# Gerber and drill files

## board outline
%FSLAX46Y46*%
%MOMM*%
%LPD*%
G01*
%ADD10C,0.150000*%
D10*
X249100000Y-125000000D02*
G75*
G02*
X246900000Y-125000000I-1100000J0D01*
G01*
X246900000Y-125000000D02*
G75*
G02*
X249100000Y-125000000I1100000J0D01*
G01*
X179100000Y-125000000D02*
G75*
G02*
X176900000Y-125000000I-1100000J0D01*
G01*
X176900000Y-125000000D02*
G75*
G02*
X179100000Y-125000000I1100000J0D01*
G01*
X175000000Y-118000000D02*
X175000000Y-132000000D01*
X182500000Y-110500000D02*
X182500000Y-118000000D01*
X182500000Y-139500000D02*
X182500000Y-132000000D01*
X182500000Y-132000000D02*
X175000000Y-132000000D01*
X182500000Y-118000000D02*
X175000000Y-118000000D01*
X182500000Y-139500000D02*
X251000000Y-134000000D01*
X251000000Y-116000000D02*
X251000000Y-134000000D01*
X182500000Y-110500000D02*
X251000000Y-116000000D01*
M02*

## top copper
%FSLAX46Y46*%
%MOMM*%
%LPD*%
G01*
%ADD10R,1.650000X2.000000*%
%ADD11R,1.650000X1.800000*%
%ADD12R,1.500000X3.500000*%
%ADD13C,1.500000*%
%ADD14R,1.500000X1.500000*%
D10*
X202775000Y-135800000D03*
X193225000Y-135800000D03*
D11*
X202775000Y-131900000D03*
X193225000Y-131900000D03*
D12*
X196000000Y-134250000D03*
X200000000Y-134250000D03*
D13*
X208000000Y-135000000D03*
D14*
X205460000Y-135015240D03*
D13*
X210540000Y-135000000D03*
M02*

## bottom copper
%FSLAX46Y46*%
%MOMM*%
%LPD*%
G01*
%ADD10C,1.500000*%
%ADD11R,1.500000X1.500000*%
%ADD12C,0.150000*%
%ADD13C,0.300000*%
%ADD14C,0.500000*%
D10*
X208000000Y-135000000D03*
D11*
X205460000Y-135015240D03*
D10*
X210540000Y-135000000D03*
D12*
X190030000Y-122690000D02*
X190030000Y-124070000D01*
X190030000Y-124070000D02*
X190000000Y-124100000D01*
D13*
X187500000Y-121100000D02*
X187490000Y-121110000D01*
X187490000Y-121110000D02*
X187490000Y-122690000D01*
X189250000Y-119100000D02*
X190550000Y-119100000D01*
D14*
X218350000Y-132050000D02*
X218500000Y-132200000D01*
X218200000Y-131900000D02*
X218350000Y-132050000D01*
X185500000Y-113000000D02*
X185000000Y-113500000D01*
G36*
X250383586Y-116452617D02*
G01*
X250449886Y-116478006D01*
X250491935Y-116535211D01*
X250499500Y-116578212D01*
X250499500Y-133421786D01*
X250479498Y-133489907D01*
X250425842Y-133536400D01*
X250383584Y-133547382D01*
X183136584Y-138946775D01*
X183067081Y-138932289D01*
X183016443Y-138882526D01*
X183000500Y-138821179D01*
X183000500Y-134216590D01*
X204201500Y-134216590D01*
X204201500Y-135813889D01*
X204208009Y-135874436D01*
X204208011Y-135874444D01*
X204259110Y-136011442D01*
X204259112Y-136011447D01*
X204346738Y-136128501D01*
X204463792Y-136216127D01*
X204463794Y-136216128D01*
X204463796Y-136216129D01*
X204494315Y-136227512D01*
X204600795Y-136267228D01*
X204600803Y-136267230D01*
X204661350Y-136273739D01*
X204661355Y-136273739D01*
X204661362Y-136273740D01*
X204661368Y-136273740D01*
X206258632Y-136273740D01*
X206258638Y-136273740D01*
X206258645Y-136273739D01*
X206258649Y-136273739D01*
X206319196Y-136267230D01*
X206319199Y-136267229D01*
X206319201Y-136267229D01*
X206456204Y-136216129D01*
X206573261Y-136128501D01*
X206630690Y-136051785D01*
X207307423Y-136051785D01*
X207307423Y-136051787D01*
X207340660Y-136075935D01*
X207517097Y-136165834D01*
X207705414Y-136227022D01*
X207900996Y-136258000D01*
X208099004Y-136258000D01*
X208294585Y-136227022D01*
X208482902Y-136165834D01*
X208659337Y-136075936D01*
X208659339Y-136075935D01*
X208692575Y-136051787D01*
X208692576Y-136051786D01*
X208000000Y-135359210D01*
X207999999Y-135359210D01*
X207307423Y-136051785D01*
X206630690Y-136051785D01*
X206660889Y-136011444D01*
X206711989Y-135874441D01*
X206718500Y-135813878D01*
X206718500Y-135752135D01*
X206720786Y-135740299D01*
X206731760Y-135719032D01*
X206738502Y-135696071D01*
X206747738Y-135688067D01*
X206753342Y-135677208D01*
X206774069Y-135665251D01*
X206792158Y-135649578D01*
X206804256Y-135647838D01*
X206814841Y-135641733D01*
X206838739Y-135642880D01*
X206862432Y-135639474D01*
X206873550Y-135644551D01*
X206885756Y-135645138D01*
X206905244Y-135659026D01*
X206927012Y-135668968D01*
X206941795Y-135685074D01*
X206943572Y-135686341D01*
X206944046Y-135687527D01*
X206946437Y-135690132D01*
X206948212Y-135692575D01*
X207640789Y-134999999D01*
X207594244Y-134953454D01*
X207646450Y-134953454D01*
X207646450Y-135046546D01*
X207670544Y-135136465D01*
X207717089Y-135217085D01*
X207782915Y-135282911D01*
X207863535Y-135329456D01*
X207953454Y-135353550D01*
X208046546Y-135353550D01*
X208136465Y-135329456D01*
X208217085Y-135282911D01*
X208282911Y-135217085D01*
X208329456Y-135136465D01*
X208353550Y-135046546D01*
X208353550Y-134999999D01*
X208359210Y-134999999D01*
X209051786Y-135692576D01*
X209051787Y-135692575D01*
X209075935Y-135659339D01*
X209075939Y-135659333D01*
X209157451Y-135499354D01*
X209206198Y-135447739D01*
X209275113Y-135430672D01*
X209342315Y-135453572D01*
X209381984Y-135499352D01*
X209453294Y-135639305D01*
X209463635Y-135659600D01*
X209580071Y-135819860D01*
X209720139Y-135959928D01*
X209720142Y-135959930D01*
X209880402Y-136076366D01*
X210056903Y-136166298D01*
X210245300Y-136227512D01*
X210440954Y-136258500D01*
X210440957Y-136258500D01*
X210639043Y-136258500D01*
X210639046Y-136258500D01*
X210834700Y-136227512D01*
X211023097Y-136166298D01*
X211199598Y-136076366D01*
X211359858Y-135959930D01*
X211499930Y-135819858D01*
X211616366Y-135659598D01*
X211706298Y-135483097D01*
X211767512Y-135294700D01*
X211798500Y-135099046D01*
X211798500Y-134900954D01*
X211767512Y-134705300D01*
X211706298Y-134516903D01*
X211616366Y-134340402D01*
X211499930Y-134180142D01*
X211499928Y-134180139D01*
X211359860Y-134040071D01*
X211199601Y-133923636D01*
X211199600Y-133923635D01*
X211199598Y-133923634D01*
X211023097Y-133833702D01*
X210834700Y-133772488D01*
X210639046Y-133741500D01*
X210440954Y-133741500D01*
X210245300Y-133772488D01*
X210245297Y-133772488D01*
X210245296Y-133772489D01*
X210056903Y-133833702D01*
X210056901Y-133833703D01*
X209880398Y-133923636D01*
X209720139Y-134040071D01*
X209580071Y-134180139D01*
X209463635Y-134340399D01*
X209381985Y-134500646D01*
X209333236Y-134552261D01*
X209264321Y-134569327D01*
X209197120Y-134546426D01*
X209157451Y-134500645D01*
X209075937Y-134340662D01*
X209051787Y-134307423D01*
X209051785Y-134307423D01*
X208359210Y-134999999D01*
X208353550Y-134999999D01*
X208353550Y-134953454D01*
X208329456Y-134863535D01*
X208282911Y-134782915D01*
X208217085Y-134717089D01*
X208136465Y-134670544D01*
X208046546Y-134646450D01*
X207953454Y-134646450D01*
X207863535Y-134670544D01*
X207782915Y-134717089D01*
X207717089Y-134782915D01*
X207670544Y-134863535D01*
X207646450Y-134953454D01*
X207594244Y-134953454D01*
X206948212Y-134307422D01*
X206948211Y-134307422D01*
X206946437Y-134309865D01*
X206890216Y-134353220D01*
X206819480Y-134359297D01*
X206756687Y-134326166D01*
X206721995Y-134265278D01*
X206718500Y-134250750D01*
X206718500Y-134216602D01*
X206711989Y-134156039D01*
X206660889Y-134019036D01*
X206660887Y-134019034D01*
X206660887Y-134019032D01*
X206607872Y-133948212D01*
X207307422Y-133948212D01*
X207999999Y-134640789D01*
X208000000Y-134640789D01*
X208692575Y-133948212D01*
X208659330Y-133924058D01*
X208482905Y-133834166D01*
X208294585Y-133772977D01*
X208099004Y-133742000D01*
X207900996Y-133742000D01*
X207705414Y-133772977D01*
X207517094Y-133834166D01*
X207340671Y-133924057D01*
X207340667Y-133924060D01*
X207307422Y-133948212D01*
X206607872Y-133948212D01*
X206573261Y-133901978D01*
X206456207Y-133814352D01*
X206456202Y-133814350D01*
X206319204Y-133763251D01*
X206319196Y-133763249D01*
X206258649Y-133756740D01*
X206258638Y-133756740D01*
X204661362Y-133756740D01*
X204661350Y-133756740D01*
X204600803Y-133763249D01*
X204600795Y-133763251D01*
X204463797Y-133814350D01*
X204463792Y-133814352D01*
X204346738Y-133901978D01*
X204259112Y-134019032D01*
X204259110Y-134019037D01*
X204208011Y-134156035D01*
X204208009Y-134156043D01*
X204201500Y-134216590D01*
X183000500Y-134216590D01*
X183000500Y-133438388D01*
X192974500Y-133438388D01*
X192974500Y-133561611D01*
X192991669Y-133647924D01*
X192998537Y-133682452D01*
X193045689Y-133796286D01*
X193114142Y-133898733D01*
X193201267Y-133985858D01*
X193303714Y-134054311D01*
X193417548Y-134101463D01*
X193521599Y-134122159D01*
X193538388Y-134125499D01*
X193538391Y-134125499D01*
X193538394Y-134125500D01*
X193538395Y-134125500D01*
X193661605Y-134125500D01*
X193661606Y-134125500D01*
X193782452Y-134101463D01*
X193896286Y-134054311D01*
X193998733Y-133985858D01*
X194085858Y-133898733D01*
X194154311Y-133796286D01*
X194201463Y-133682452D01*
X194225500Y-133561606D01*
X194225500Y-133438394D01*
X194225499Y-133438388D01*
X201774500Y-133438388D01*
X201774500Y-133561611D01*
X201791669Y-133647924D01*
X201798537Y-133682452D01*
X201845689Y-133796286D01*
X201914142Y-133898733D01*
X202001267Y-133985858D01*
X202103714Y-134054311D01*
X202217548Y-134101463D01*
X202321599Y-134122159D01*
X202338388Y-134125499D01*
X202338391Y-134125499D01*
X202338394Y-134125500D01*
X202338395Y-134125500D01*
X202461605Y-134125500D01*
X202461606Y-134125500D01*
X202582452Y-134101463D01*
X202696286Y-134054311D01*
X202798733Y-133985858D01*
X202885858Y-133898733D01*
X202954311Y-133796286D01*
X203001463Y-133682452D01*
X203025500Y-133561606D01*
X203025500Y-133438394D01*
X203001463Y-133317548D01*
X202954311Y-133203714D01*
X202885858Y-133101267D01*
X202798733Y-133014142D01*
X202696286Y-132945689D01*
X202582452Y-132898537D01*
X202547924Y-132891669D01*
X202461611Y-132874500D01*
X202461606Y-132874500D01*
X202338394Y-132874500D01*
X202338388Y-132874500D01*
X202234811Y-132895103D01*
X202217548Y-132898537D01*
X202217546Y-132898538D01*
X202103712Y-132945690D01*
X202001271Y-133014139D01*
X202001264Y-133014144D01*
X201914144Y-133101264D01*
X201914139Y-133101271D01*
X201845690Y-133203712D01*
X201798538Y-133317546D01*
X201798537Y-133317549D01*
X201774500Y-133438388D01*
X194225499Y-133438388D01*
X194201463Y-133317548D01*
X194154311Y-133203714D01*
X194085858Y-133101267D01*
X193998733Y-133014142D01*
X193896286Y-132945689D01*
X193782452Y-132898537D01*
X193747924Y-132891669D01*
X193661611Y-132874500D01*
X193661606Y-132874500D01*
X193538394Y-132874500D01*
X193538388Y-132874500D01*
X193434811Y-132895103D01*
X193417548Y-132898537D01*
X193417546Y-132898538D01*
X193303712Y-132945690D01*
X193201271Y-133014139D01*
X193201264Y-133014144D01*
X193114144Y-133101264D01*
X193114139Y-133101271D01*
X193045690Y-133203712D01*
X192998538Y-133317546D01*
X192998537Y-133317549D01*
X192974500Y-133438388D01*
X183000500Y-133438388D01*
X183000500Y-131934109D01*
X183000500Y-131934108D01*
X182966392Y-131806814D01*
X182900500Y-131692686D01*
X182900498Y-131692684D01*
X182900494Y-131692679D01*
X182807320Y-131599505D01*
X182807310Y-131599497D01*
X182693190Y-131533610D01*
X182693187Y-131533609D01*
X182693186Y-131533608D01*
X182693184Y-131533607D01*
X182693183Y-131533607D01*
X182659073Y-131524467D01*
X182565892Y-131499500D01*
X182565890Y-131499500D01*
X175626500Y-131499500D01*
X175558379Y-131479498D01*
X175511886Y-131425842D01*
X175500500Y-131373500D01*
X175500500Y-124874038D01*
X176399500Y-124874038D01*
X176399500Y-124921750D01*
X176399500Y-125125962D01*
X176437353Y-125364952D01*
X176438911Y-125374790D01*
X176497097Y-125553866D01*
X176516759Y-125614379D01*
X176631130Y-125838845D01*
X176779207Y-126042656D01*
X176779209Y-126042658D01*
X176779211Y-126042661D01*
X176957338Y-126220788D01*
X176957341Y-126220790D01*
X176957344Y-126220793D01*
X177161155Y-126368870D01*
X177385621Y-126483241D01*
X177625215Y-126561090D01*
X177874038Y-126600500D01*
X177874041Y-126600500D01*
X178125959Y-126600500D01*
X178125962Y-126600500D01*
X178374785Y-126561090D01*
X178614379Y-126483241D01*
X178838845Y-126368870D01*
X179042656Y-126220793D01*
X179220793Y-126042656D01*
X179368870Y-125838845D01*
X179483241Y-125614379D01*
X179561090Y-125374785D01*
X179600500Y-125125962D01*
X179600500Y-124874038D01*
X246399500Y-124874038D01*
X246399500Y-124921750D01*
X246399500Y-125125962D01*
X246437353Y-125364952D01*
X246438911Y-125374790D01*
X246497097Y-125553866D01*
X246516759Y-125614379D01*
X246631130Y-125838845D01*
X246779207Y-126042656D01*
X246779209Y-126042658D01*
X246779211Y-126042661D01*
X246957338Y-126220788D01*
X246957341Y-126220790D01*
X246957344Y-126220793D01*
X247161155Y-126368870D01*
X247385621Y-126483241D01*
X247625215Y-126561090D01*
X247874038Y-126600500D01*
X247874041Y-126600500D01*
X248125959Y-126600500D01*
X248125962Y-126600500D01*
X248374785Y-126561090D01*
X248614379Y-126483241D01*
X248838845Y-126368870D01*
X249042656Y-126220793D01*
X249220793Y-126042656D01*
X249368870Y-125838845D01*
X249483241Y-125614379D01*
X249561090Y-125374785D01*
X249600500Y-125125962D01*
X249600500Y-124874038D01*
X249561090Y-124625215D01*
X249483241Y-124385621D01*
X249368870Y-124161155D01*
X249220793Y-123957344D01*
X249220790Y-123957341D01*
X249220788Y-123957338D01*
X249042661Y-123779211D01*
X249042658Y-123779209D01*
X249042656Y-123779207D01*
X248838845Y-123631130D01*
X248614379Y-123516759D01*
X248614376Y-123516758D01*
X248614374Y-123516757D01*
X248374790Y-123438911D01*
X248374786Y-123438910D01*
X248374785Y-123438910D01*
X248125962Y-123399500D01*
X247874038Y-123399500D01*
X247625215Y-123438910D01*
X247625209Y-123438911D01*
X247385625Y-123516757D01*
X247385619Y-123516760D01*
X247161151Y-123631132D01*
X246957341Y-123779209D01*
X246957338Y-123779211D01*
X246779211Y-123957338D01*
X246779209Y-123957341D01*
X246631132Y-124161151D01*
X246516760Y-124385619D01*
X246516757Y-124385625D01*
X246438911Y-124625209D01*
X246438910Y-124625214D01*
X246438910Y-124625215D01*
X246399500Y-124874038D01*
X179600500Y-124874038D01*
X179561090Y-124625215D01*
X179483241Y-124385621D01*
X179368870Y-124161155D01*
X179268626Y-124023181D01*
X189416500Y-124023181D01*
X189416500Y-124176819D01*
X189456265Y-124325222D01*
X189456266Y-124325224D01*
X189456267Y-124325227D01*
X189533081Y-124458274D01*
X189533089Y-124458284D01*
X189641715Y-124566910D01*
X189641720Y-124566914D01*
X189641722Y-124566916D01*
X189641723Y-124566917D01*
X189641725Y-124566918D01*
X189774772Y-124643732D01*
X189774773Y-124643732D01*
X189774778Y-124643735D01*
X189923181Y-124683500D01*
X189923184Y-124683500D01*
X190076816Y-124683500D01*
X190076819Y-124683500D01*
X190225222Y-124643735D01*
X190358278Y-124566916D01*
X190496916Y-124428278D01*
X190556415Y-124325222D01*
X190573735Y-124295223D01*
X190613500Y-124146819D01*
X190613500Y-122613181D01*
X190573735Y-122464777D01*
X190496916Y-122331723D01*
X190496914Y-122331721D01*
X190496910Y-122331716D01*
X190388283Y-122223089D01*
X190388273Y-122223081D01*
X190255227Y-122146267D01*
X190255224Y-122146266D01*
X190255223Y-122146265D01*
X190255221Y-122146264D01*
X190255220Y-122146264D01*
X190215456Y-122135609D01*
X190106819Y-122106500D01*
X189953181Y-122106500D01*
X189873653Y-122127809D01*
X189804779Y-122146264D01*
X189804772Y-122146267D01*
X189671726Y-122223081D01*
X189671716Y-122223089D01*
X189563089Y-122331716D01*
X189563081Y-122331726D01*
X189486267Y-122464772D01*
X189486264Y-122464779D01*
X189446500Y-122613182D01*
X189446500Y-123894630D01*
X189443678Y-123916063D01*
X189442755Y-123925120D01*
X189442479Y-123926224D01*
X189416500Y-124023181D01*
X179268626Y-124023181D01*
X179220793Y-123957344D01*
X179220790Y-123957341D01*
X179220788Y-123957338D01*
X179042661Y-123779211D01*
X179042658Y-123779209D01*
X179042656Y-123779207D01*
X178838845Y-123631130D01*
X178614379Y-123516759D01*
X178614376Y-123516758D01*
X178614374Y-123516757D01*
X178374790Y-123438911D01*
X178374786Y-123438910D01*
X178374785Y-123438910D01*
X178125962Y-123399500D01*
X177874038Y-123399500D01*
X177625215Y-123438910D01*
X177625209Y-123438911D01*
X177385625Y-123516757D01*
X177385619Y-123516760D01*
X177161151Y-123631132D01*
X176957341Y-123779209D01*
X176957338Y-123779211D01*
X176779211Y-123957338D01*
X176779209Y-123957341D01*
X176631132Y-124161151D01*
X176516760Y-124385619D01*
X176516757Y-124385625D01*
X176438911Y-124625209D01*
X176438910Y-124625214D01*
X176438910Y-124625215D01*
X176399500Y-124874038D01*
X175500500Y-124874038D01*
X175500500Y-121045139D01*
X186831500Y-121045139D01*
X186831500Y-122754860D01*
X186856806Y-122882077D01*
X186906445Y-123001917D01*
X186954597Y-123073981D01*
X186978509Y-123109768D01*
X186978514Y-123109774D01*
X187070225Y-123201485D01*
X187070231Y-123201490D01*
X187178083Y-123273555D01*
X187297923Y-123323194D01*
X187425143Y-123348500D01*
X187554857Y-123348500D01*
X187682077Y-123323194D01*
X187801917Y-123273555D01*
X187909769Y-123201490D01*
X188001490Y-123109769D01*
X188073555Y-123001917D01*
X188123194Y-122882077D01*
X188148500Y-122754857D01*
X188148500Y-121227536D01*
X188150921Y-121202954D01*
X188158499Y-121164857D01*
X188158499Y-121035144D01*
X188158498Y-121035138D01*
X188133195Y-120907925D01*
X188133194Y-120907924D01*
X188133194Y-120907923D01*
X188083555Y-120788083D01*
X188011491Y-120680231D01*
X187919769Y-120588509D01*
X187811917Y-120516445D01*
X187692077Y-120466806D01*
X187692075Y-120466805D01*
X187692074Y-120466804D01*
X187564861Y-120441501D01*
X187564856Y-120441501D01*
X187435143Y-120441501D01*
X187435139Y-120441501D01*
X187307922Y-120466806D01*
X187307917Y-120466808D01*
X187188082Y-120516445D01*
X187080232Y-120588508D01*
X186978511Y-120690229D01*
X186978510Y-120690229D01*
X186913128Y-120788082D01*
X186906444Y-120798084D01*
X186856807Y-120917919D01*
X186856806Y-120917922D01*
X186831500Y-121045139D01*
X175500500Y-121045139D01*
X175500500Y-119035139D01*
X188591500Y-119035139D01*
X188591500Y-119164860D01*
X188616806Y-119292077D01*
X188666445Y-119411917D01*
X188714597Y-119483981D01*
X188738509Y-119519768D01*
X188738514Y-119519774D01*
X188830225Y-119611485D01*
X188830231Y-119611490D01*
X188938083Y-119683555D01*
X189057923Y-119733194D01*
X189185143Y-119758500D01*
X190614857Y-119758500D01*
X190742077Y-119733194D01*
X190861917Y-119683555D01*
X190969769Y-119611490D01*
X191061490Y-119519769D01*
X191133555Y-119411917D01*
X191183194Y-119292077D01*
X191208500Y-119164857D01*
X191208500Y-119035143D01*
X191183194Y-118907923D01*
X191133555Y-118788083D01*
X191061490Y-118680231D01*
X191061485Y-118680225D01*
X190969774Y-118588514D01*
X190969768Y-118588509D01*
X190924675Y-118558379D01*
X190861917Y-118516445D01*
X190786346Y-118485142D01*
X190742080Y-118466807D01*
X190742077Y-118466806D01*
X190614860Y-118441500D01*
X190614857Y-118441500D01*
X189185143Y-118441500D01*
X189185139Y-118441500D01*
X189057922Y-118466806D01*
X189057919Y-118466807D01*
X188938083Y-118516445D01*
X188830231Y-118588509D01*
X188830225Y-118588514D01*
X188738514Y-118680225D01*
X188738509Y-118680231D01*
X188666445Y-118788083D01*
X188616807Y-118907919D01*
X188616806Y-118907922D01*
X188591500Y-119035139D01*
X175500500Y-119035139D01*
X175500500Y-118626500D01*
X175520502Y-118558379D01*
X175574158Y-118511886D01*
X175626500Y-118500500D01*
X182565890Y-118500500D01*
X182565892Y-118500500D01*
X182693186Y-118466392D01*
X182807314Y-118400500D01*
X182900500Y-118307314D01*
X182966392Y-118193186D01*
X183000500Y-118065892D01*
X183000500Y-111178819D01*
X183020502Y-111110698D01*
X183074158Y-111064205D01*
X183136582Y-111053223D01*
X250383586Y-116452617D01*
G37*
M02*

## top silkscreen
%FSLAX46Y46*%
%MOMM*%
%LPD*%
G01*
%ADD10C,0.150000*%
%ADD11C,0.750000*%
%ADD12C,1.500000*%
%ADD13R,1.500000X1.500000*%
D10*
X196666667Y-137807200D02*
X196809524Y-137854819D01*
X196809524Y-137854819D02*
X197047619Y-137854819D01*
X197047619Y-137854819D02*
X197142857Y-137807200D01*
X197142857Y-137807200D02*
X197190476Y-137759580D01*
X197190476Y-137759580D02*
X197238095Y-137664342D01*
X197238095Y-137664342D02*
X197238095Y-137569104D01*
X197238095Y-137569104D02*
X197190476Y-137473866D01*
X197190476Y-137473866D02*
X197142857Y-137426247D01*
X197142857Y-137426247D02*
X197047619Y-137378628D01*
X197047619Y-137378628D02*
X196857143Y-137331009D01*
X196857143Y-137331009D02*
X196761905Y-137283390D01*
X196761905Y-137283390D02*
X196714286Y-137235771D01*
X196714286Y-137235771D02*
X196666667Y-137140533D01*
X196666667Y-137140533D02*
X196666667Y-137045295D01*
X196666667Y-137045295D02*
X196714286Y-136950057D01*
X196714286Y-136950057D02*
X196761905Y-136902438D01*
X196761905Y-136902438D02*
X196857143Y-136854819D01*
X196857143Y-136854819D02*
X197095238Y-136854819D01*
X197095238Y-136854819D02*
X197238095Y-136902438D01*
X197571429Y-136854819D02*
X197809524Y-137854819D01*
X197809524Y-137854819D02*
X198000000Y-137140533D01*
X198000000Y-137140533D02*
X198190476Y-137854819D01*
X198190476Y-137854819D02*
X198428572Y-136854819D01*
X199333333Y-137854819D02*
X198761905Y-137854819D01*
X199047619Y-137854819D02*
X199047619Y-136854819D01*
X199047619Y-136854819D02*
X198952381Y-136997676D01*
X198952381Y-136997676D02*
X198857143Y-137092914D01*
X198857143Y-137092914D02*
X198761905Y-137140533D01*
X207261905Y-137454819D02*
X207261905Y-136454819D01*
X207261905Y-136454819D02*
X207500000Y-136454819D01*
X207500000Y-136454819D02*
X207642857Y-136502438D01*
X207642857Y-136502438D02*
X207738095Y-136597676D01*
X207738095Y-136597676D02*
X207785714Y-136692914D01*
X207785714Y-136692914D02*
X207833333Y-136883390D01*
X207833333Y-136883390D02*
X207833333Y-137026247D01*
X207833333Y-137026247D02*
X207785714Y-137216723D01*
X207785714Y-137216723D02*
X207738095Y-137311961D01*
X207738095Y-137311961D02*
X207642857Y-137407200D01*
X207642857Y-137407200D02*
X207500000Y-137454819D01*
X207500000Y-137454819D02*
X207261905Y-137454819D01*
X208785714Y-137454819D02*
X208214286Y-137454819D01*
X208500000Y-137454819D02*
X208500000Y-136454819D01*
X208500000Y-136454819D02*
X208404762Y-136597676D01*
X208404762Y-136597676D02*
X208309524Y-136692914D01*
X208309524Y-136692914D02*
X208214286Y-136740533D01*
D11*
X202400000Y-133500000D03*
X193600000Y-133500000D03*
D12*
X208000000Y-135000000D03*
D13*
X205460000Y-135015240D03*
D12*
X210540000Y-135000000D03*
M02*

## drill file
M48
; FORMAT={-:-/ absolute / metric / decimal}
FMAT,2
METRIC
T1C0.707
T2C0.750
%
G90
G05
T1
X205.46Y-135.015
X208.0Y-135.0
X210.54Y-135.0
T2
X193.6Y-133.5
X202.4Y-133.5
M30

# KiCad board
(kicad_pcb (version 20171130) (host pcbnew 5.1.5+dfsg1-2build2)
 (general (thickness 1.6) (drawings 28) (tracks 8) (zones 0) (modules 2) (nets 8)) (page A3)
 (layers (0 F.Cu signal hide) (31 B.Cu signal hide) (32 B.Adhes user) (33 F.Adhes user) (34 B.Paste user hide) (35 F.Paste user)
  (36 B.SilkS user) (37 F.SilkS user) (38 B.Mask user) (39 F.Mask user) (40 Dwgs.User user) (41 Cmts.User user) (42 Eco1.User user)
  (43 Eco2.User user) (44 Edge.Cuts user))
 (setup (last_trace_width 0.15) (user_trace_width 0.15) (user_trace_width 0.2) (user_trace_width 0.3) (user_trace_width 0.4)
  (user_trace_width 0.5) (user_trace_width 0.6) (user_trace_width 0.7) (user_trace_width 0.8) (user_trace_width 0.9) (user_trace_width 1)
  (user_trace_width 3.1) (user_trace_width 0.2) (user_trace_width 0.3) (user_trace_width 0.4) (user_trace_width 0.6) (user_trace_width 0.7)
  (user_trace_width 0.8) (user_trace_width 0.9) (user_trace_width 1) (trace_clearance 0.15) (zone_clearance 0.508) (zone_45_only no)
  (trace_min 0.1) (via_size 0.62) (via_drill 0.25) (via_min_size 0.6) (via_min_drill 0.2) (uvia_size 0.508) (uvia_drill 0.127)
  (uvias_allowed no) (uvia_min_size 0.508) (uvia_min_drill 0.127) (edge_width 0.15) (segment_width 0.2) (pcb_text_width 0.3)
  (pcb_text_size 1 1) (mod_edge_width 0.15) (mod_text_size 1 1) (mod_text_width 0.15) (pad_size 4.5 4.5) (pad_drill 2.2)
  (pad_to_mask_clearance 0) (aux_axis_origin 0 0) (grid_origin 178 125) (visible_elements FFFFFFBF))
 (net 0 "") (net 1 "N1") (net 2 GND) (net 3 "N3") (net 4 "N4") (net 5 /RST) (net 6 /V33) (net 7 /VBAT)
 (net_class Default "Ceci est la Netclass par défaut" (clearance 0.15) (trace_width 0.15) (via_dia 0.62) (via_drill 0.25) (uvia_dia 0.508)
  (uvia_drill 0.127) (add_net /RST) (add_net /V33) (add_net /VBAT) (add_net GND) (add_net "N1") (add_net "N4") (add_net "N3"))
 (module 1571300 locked (layer F.Cu) (at 198 133.5)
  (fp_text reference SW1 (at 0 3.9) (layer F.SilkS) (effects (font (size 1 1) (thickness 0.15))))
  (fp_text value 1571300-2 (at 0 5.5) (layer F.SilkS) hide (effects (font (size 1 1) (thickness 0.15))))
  (pad "" np_thru_hole circle (at 4.4 0) (size 0.75 0.75) (drill 0.75) (layers *.Cu *.Mask F.SilkS))
  (pad "" np_thru_hole circle (at -4.4 0) (size 0.75 0.75) (drill 0.75) (layers *.Cu *.Mask F.SilkS))
  (pad "" smd rect (at 4.775 2.3) (size 1.65 2) (layers F.Cu F.Paste F.Mask))
  (pad "" smd rect (at -4.775 2.3) (size 1.65 2) (layers F.Cu F.Paste F.Mask))
  (pad "" smd rect (at 4.775 -1.6) (size 1.65 1.8) (layers F.Cu F.Paste F.Mask))
  (pad "" smd rect (at -4.775 -1.6) (size 1.65 1.8) (layers F.Cu F.Paste F.Mask))
  (pad 1 smd rect (at -2 0.75) (size 1.5 3.5) (layers F.Cu F.Paste F.Mask) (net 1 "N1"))
  (pad 2 smd rect (at 2 0.75) (size 1.5 3.5) (layers F.Cu F.Paste F.Mask) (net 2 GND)))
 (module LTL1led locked (layer F.Cu) (at 208 135 180)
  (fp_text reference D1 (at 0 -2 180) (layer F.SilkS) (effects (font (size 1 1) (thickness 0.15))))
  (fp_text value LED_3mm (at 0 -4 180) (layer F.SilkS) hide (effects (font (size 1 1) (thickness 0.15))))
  (pad 2 thru_hole circle (at 0 0 180) (size 1.5 1.5) (drill 0.7071) (layers *.Cu *.Mask F.SilkS) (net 2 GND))
  (pad 1 thru_hole rect (at 2.54 -0.01524 180) (size 1.5 1.5) (drill 0.7071) (layers *.Cu *.Mask F.SilkS) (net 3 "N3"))
  (pad 3 thru_hole circle (at -2.54 0 180) (size 1.5 1.5) (drill 0.7071) (layers *.Cu *.Mask F.SilkS) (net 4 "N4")))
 (gr_circle (center 248 125) (end 249.1 125) (layer Edge.Cuts) (width 0.15))
 (gr_circle (center 178 125) (end 179.1 125) (layer Edge.Cuts) (width 0.15))
 (gr_line (start 175 118) (end 175 132) (angle 90) (layer Edge.Cuts) (width 0.15))
 (gr_line (start 182.5 110.5) (end 182.5 118) (angle 90) (layer Edge.Cuts) (width 0.15))
 (gr_line (start 182.5 139.5) (end 182.5 132) (angle 90) (layer Edge.Cuts) (width 0.15))
 (gr_line (start 182.5 132) (end 175 132) (angle 90) (layer Edge.Cuts) (width 0.15))
 (gr_line (start 182.5 118) (end 175 118) (angle 90) (layer Edge.Cuts) (width 0.15))
 (gr_line (start 182.5 139.5) (end 251 134) (angle 90) (layer Edge.Cuts) (width 0.15))
 (gr_line (start 251 116) (end 251 134) (angle 90) (layer Edge.Cuts) (width 0.15))
 (gr_line (start 182.5 110.5) (end 251 116) (angle 90) (layer Edge.Cuts) (width 0.15))
 (segment (start 190.03 122.69) (end 190.03 124.07) (width 0.15) (layer B.Cu) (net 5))
 (segment (start 190.03 124.07) (end 190 124.1) (width 0.15) (layer B.Cu) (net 5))
 (segment (start 187.5 121.1) (end 187.49 121.11) (width 0.3) (layer B.Cu) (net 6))
 (segment (start 187.49 121.11) (end 187.49 122.69) (width 0.3) (layer B.Cu) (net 6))
 (segment (start 189.25 119.1) (end 190.55 119.1) (width 0.3) (layer B.Cu) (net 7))
 (segment (start 218.35 132.05) (end 218.5 132.2) (width 0.5) (layer B.Cu) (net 2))
 (segment (start 218.2 131.9) (end 218.35 132.05) (width 0.5) (layer B.Cu) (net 2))
 (segment (start 185.5 113) (end 185 113.5) (width 0.5) (layer B.Cu) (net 2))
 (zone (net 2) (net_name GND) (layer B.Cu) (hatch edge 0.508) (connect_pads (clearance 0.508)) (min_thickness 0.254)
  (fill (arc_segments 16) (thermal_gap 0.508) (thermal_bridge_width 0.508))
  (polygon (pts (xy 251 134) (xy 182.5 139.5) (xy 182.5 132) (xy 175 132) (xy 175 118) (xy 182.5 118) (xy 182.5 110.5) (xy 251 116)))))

